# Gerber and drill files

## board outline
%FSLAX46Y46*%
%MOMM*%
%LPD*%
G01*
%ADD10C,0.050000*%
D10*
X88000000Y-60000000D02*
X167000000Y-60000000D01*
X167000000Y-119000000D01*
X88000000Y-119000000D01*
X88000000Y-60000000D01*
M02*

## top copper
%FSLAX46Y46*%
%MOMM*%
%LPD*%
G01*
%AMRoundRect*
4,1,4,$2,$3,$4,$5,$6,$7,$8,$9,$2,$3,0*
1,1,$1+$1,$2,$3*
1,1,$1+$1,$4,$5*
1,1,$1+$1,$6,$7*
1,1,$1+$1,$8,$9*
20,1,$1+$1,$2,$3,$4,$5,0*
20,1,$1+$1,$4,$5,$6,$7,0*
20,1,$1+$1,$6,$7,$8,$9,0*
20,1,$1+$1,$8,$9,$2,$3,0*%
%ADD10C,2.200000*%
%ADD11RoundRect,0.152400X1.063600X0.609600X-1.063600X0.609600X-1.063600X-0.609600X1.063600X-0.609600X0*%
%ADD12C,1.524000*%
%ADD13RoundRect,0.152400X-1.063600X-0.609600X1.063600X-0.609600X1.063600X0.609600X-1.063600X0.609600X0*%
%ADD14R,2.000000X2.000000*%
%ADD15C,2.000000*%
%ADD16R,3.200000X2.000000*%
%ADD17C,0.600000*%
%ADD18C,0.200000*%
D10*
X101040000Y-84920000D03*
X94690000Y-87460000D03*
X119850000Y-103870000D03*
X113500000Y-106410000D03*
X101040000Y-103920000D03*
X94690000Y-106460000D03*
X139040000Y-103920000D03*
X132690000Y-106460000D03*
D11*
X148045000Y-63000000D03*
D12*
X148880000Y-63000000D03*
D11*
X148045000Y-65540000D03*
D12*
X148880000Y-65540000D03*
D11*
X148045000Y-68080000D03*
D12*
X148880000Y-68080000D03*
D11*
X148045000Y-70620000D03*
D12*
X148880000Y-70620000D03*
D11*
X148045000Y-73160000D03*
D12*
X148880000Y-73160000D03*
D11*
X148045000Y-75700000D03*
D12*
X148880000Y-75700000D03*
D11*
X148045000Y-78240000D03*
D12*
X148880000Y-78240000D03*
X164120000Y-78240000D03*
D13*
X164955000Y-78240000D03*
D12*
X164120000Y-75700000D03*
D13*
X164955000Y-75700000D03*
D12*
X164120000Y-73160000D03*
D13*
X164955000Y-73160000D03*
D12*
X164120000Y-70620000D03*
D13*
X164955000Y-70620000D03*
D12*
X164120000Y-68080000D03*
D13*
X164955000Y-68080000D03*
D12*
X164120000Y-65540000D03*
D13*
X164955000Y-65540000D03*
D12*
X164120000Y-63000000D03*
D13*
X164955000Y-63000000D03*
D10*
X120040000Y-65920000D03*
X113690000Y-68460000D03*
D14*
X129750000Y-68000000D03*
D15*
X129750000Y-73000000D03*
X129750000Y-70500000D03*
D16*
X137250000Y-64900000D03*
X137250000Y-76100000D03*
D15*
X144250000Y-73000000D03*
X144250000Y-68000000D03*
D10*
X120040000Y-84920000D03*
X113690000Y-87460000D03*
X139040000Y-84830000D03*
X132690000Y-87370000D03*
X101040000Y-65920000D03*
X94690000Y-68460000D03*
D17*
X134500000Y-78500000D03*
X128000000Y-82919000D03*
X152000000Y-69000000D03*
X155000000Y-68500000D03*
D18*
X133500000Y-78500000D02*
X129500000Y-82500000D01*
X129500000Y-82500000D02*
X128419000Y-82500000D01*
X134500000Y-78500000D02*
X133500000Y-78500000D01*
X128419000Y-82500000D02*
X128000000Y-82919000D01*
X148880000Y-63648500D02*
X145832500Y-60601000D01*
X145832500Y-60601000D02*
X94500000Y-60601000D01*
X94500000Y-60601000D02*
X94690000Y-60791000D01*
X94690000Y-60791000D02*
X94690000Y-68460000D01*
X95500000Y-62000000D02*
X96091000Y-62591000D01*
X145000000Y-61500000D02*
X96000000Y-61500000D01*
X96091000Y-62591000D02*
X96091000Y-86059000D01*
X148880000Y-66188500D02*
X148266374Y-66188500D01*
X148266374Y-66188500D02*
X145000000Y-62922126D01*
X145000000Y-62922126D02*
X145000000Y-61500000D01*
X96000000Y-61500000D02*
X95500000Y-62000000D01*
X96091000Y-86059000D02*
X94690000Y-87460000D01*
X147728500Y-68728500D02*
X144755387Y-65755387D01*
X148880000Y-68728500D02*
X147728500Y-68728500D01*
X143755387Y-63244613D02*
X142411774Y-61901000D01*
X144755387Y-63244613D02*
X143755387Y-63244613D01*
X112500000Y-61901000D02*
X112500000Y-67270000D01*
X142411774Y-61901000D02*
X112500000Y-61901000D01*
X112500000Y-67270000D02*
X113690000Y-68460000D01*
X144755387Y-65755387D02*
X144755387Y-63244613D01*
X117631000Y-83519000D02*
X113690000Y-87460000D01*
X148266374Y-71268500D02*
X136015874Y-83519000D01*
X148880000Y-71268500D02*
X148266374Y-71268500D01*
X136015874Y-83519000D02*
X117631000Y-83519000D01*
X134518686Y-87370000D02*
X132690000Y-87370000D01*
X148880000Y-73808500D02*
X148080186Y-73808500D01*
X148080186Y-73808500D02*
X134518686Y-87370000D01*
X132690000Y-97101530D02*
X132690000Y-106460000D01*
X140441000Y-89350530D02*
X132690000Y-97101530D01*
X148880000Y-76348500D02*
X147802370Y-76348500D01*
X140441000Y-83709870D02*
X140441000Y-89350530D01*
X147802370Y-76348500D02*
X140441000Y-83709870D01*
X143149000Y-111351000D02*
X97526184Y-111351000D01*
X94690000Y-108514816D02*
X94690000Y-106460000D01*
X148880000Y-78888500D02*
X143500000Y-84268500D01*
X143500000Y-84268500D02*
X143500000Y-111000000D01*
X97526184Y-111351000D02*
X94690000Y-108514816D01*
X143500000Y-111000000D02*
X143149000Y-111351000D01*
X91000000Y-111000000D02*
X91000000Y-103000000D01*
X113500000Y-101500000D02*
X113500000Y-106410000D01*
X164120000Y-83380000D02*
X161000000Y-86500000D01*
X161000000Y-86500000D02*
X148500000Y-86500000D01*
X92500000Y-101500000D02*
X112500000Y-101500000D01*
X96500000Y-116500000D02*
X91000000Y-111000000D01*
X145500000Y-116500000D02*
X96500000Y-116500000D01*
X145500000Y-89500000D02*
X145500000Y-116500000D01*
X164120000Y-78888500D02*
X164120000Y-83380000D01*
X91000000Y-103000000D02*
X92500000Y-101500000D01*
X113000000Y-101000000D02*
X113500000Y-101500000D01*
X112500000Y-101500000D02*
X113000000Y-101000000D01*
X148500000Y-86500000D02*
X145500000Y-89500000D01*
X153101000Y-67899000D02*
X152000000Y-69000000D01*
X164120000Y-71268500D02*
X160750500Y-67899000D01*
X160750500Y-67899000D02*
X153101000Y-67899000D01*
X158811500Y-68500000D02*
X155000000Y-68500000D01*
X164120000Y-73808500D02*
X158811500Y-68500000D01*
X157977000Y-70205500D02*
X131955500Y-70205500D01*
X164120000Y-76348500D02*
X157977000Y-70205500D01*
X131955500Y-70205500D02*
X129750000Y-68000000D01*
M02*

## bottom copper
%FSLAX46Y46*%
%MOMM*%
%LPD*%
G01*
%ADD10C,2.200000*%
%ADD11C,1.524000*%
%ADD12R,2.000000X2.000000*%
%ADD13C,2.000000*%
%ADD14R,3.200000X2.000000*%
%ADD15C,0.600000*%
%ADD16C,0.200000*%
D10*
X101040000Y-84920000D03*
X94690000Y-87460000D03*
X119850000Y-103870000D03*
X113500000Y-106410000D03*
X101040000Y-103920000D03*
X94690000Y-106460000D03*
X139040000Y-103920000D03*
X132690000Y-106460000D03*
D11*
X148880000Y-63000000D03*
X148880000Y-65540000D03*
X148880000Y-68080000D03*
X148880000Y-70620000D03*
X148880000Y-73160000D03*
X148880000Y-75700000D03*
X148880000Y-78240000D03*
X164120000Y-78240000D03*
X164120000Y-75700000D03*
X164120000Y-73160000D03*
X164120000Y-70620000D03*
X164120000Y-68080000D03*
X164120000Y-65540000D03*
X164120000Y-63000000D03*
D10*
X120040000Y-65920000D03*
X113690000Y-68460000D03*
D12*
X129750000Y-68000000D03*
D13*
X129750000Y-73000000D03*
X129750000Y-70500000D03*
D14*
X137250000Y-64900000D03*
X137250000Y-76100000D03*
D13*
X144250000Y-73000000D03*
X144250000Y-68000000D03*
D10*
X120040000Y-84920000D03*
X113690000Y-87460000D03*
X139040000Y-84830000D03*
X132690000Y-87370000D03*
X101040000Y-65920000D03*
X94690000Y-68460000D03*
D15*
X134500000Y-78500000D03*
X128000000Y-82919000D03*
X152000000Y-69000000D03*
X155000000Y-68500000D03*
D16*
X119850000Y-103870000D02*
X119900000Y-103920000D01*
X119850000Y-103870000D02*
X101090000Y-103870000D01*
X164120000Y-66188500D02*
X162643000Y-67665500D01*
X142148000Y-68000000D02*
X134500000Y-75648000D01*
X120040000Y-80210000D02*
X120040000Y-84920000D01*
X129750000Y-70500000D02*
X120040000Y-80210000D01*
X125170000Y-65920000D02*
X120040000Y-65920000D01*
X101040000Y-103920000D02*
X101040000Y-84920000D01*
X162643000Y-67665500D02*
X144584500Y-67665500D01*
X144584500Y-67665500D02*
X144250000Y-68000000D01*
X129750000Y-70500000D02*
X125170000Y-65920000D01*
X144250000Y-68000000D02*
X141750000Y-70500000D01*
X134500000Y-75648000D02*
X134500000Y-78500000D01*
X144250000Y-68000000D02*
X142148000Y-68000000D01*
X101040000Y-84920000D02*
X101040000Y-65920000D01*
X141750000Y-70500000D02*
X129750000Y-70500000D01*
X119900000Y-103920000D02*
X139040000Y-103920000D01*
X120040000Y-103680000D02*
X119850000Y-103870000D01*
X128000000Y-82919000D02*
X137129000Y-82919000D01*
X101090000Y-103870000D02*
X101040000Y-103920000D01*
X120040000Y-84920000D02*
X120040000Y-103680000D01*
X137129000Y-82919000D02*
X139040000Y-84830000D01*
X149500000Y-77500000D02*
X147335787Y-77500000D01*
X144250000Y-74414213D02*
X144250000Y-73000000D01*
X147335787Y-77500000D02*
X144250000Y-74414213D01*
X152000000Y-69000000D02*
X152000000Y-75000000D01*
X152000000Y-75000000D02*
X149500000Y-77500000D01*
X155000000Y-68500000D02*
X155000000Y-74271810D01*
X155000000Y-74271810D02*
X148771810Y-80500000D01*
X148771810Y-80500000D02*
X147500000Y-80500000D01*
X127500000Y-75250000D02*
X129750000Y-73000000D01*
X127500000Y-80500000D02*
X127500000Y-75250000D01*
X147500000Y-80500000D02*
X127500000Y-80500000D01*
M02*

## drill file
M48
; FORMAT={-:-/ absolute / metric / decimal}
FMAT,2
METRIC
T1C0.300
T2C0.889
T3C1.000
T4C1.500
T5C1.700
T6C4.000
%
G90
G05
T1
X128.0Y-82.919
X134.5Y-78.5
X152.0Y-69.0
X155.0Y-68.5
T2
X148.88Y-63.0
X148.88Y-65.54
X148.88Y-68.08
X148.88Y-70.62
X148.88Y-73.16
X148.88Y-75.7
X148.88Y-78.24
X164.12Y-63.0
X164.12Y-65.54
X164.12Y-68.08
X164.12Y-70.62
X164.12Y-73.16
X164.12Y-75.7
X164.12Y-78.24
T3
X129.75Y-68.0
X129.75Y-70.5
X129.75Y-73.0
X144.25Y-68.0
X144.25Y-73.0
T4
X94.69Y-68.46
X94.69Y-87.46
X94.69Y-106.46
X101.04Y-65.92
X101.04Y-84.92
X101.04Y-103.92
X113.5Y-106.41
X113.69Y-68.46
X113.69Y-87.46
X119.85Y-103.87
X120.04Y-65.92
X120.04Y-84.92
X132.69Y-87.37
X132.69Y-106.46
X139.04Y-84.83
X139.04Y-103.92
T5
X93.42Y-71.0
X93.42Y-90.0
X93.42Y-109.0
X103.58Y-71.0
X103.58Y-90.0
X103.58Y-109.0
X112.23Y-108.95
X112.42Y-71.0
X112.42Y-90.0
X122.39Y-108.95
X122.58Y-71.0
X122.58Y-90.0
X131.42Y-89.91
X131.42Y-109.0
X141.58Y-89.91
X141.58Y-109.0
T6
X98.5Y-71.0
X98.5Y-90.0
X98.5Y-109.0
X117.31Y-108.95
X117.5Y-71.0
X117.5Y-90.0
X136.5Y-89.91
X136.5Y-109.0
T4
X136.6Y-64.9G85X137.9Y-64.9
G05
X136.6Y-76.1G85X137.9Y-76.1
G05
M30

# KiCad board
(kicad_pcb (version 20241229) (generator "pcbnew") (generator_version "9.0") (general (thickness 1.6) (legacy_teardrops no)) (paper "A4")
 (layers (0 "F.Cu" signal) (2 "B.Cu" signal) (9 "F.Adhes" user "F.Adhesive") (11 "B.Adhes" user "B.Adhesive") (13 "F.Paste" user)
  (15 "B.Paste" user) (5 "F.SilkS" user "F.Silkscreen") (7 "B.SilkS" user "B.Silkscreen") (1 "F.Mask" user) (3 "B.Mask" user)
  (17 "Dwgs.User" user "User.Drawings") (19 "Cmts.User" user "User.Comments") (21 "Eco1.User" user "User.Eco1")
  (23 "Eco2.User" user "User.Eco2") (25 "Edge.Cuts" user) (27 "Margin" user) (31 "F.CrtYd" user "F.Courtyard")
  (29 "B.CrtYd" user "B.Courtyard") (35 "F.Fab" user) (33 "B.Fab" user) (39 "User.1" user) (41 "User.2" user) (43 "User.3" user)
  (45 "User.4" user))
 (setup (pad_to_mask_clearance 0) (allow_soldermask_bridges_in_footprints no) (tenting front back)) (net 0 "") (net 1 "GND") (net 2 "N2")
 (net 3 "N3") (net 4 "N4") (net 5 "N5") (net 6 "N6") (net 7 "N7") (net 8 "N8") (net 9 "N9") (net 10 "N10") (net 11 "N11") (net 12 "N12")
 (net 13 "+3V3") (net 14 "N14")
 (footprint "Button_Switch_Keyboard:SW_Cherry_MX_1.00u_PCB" (layer "F.Cu") (at 101.04 84.92)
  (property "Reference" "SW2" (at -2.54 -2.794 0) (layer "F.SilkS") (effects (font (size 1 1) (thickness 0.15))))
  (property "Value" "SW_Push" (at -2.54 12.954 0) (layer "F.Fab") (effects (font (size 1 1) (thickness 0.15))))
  (pad "" np_thru_hole circle (at -7.62 5.08) (size 1.7 1.7) (drill 1.7) (layers "*.Cu" "*.Mask"))
  (pad "" np_thru_hole circle (at -2.54 5.08) (size 4 4) (drill 4) (layers "*.Cu" "*.Mask"))
  (pad "" np_thru_hole circle (at 2.54 5.08) (size 1.7 1.7) (drill 1.7) (layers "*.Cu" "*.Mask"))
  (pad "1" thru_hole circle (at 0 0) (size 2.2 2.2) (drill 1.5) (layers "*.Cu" "*.Mask") (remove_unused_layers no) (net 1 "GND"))
  (pad "2" thru_hole circle (at -6.35 2.54) (size 2.2 2.2) (drill 1.5) (layers "*.Cu" "*.Mask") (remove_unused_layers no) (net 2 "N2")))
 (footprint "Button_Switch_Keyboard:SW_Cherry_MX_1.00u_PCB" (layer "F.Cu") (at 119.85 103.87)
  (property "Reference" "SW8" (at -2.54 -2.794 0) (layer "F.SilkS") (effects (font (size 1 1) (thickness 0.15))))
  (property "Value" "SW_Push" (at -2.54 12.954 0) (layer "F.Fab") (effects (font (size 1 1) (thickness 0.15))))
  (pad "" np_thru_hole circle (at -7.62 5.08) (size 1.7 1.7) (drill 1.7) (layers "*.Cu" "*.Mask"))
  (pad "" np_thru_hole circle (at -2.54 5.08) (size 4 4) (drill 4) (layers "*.Cu" "*.Mask"))
  (pad "" np_thru_hole circle (at 2.54 5.08) (size 1.7 1.7) (drill 1.7) (layers "*.Cu" "*.Mask"))
  (pad "1" thru_hole circle (at 0 0) (size 2.2 2.2) (drill 1.5) (layers "*.Cu" "*.Mask") (remove_unused_layers no) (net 1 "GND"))
  (pad "2" thru_hole circle (at -6.35 2.54) (size 2.2 2.2) (drill 1.5) (layers "*.Cu" "*.Mask") (remove_unused_layers no) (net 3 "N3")))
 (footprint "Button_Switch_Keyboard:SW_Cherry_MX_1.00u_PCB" (layer "F.Cu") (at 101.04 103.92)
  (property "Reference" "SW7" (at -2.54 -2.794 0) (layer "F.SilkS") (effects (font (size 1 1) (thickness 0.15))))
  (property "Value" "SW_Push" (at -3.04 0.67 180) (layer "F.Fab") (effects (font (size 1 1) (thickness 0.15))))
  (pad "" np_thru_hole circle (at -7.62 5.08) (size 1.7 1.7) (drill 1.7) (layers "*.Cu" "*.Mask"))
  (pad "" np_thru_hole circle (at -2.54 5.08) (size 4 4) (drill 4) (layers "*.Cu" "*.Mask"))
  (pad "" np_thru_hole circle (at 2.54 5.08) (size 1.7 1.7) (drill 1.7) (layers "*.Cu" "*.Mask"))
  (pad "1" thru_hole circle (at 0 0) (size 2.2 2.2) (drill 1.5) (layers "*.Cu" "*.Mask") (remove_unused_layers no) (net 1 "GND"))
  (pad "2" thru_hole circle (at -6.35 2.54) (size 2.2 2.2) (drill 1.5) (layers "*.Cu" "*.Mask") (remove_unused_layers no) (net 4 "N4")))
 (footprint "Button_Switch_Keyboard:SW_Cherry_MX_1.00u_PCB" (layer "F.Cu") (at 139.04 103.92)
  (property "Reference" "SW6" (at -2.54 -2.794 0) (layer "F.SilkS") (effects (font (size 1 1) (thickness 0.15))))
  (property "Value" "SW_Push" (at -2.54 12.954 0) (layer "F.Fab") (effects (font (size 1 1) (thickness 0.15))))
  (pad "" np_thru_hole circle (at -7.62 5.08) (size 1.7 1.7) (drill 1.7) (layers "*.Cu" "*.Mask"))
  (pad "" np_thru_hole circle (at -2.54 5.08) (size 4 4) (drill 4) (layers "*.Cu" "*.Mask"))
  (pad "" np_thru_hole circle (at 2.54 5.08) (size 1.7 1.7) (drill 1.7) (layers "*.Cu" "*.Mask"))
  (pad "1" thru_hole circle (at 0 0) (size 2.2 2.2) (drill 1.5) (layers "*.Cu" "*.Mask") (remove_unused_layers no) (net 1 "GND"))
  (pad "2" thru_hole circle (at -6.35 2.54) (size 2.2 2.2) (drill 1.5) (layers "*.Cu" "*.Mask") (remove_unused_layers no) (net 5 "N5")))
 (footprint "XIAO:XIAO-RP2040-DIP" (layer "F.Cu") (at 156.5 70.62)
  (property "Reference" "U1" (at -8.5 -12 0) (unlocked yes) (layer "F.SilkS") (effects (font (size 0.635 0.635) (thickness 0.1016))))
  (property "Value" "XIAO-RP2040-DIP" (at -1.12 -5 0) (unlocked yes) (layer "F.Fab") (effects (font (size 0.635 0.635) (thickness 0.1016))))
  (pad "1" smd roundrect (at -8.455 -7.62 180) (size 2.432 1.524) (layers "F.Cu" "F.Mask") (roundrect_rratio 0.1) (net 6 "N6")
   (thermal_bridge_angle 45))
  (pad "1" thru_hole circle (at -7.62 -7.62 180) (size 1.524 1.524) (drill 0.889) (layers "*.Cu" "*.Mask") (remove_unused_layers no)
   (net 6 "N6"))
  (pad "2" smd roundrect (at -8.455 -5.08 180) (size 2.432 1.524) (layers "F.Cu" "F.Mask") (roundrect_rratio 0.1) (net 2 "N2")
   (thermal_bridge_angle 45))
  (pad "2" thru_hole circle (at -7.62 -5.08 180) (size 1.524 1.524) (drill 0.889) (layers "*.Cu" "*.Mask") (remove_unused_layers no)
   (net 2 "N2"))
  (pad "3" smd roundrect (at -8.455 -2.54 180) (size 2.432 1.524) (layers "F.Cu" "F.Mask") (roundrect_rratio 0.1) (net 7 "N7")
   (thermal_bridge_angle 45))
  (pad "3" thru_hole circle (at -7.62 -2.54 180) (size 1.524 1.524) (drill 0.889) (layers "*.Cu" "*.Mask") (remove_unused_layers no)
   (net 7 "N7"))
  (pad "4" smd roundrect (at -8.455 0 180) (size 2.432 1.524) (layers "F.Cu" "F.Mask") (roundrect_rratio 0.1) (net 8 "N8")
   (thermal_bridge_angle 45))
  (pad "4" thru_hole circle (at -7.62 0 180) (size 1.524 1.524) (drill 0.889) (layers "*.Cu" "*.Mask") (remove_unused_layers no)
   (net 8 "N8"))
  (pad "5" smd roundrect (at -8.455 2.54 180) (size 2.432 1.524) (layers "F.Cu" "F.Mask") (roundrect_rratio 0.1) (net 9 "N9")
   (thermal_bridge_angle 45))
  (pad "5" thru_hole circle (at -7.62 2.54 180) (size 1.524 1.524) (drill 0.889) (layers "*.Cu" "*.Mask") (remove_unused_layers no)
   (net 9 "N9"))
  (pad "6" smd roundrect (at -8.455 5.08 180) (size 2.432 1.524) (layers "F.Cu" "F.Mask") (roundrect_rratio 0.1) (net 5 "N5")
   (thermal_bridge_angle 45))
  (pad "6" thru_hole circle (at -7.62 5.08 180) (size 1.524 1.524) (drill 0.889) (layers "*.Cu" "*.Mask") (remove_unused_layers no)
   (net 5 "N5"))
  (pad "7" smd roundrect (at -8.455 7.62 180) (size 2.432 1.524) (layers "F.Cu" "F.Mask") (roundrect_rratio 0.1) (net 4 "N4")
   (thermal_bridge_angle 45))
  (pad "7" thru_hole circle (at -7.62 7.62 180) (size 1.524 1.524) (drill 0.889) (layers "*.Cu" "*.Mask") (remove_unused_layers no)
   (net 4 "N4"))
  (pad "8" thru_hole circle (at 7.62 7.62) (size 1.524 1.524) (drill 0.889) (layers "*.Cu" "*.Mask") (remove_unused_layers no) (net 3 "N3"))
  (pad "8" smd roundrect (at 8.455 7.62) (size 2.432 1.524) (layers "F.Cu" "F.Mask") (roundrect_rratio 0.1) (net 3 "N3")
   (thermal_bridge_angle 45))
  (pad "9" thru_hole circle (at 7.62 5.08) (size 1.524 1.524) (drill 0.889) (layers "*.Cu" "*.Mask") (remove_unused_layers no)
   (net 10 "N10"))
  (pad "9" smd roundrect (at 8.455 5.08) (size 2.432 1.524) (layers "F.Cu" "F.Mask") (roundrect_rratio 0.1) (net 10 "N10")
   (thermal_bridge_angle 45))
  (pad "10" thru_hole circle (at 7.62 2.54) (size 1.524 1.524) (drill 0.889) (layers "*.Cu" "*.Mask") (remove_unused_layers no)
   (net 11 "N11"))
  (pad "10" smd roundrect (at 8.455 2.54) (size 2.432 1.524) (layers "F.Cu" "F.Mask") (roundrect_rratio 0.1) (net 11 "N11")
   (thermal_bridge_angle 45))
  (pad "11" thru_hole circle (at 7.62 0) (size 1.524 1.524) (drill 0.889) (layers "*.Cu" "*.Mask") (remove_unused_layers no) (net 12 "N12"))
  (pad "11" smd roundrect (at 8.455 0) (size 2.432 1.524) (layers "F.Cu" "F.Mask") (roundrect_rratio 0.1) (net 12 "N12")
   (thermal_bridge_angle 45))
  (pad "12" thru_hole circle (at 7.62 -2.54) (size 1.524 1.524) (drill 0.889) (layers "*.Cu" "*.Mask") (remove_unused_layers no)
   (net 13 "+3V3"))
  (pad "12" smd roundrect (at 8.455 -2.54) (size 2.432 1.524) (layers "F.Cu" "F.Mask") (roundrect_rratio 0.1) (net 13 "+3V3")
   (thermal_bridge_angle 45))
  (pad "13" thru_hole circle (at 7.62 -5.08) (size 1.524 1.524) (drill 0.889) (layers "*.Cu" "*.Mask") (remove_unused_layers no)
   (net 1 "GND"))
  (pad "13" smd roundrect (at 8.455 -5.08) (size 2.432 1.524) (layers "F.Cu" "F.Mask") (roundrect_rratio 0.1) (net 1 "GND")
   (thermal_bridge_angle 45))
  (pad "14" thru_hole circle (at 7.62 -7.62) (size 1.524 1.524) (drill 0.889) (layers "*.Cu" "*.Mask") (remove_unused_layers no)
   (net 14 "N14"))
  (pad "14" smd roundrect (at 8.455 -7.62) (size 2.432 1.524) (layers "F.Cu" "F.Mask") (roundrect_rratio 0.1) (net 14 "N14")
   (thermal_bridge_angle 45)))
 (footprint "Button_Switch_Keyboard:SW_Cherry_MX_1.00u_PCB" (layer "F.Cu") (at 120.04 65.92)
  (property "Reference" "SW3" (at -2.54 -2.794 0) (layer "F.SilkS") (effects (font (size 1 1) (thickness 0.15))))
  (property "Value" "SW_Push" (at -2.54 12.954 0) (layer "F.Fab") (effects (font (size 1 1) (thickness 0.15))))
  (pad "" np_thru_hole circle (at -7.62 5.08) (size 1.7 1.7) (drill 1.7) (layers "*.Cu" "*.Mask"))
  (pad "" np_thru_hole circle (at -2.54 5.08) (size 4 4) (drill 4) (layers "*.Cu" "*.Mask"))
  (pad "" np_thru_hole circle (at 2.54 5.08) (size 1.7 1.7) (drill 1.7) (layers "*.Cu" "*.Mask"))
  (pad "1" thru_hole circle (at 0 0) (size 2.2 2.2) (drill 1.5) (layers "*.Cu" "*.Mask") (remove_unused_layers no) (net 1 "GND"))
  (pad "2" thru_hole circle (at -6.35 2.54) (size 2.2 2.2) (drill 1.5) (layers "*.Cu" "*.Mask") (remove_unused_layers no) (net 7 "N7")))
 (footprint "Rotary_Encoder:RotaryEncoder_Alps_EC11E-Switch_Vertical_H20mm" (layer "F.Cu") (at 129.75 68)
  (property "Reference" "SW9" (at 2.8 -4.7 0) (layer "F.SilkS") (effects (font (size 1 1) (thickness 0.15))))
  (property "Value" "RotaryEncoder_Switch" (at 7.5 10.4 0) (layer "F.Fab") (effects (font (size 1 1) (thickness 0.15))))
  (pad "A" thru_hole rect (at 0 0) (size 2 2) (drill 1) (layers "*.Cu" "*.Mask") (remove_unused_layers no) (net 10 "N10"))
  (pad "B" thru_hole circle (at 0 5) (size 2 2) (drill 1) (layers "*.Cu" "*.Mask") (remove_unused_layers no) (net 11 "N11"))
  (pad "C" thru_hole circle (at 0 2.5) (size 2 2) (drill 1) (layers "*.Cu" "*.Mask") (remove_unused_layers no) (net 1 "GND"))
  (pad "MP" thru_hole rect (at 7.5 -3.1) (size 3.2 2) (drill oval 2.8 1.5) (layers "*.Cu" "*.Mask") (remove_unused_layers no))
  (pad "MP" thru_hole rect (at 7.5 8.1) (size 3.2 2) (drill oval 2.8 1.5) (layers "*.Cu" "*.Mask") (remove_unused_layers no))
  (pad "S1" thru_hole circle (at 14.5 5) (size 2 2) (drill 1) (layers "*.Cu" "*.Mask") (remove_unused_layers no) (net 12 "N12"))
  (pad "S2" thru_hole circle (at 14.5 0) (size 2 2) (drill 1) (layers "*.Cu" "*.Mask") (remove_unused_layers no) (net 1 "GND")))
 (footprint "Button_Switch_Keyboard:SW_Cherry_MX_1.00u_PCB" (layer "F.Cu") (at 120.04 84.92)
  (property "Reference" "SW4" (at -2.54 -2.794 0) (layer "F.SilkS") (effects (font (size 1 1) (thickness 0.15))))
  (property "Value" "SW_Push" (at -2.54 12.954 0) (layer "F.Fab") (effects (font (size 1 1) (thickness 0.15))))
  (pad "" np_thru_hole circle (at -7.62 5.08) (size 1.7 1.7) (drill 1.7) (layers "*.Cu" "*.Mask"))
  (pad "" np_thru_hole circle (at -2.54 5.08) (size 4 4) (drill 4) (layers "*.Cu" "*.Mask"))
  (pad "" np_thru_hole circle (at 2.54 5.08) (size 1.7 1.7) (drill 1.7) (layers "*.Cu" "*.Mask"))
  (pad "1" thru_hole circle (at 0 0) (size 2.2 2.2) (drill 1.5) (layers "*.Cu" "*.Mask") (remove_unused_layers no) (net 1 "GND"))
  (pad "2" thru_hole circle (at -6.35 2.54) (size 2.2 2.2) (drill 1.5) (layers "*.Cu" "*.Mask") (remove_unused_layers no) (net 8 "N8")))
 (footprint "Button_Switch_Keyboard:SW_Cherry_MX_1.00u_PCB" (layer "F.Cu") (at 139.04 84.83)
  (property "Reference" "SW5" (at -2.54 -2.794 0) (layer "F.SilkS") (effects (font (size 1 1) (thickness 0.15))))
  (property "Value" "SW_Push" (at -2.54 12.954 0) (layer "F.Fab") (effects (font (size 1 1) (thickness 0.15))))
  (pad "" np_thru_hole circle (at -7.62 5.08) (size 1.7 1.7) (drill 1.7) (layers "*.Cu" "*.Mask"))
  (pad "" np_thru_hole circle (at -2.54 5.08) (size 4 4) (drill 4) (layers "*.Cu" "*.Mask"))
  (pad "" np_thru_hole circle (at 2.54 5.08) (size 1.7 1.7) (drill 1.7) (layers "*.Cu" "*.Mask"))
  (pad "1" thru_hole circle (at 0 0) (size 2.2 2.2) (drill 1.5) (layers "*.Cu" "*.Mask") (remove_unused_layers no) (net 1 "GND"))
  (pad "2" thru_hole circle (at -6.35 2.54) (size 2.2 2.2) (drill 1.5) (layers "*.Cu" "*.Mask") (remove_unused_layers no) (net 9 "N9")))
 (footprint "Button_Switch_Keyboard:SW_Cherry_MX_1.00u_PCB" (layer "F.Cu") (at 101.04 65.92)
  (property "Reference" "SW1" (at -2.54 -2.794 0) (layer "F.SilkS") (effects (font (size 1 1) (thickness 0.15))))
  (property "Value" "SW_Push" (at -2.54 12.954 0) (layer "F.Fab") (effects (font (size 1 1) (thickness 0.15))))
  (pad "" np_thru_hole circle (at -7.62 5.08) (size 1.7 1.7) (drill 1.7) (layers "*.Cu" "*.Mask"))
  (pad "" np_thru_hole circle (at -2.54 5.08) (size 4 4) (drill 4) (layers "*.Cu" "*.Mask"))
  (pad "" np_thru_hole circle (at 2.54 5.08) (size 1.7 1.7) (drill 1.7) (layers "*.Cu" "*.Mask"))
  (pad "1" thru_hole circle (at 0 0) (size 2.2 2.2) (drill 1.5) (layers "*.Cu" "*.Mask") (remove_unused_layers no) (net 1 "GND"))
  (pad "2" thru_hole circle (at -6.35 2.54) (size 2.2 2.2) (drill 1.5) (layers "*.Cu" "*.Mask") (remove_unused_layers no) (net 6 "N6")))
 (gr_rect (start 88 60) (end 167 119) (stroke (width 0.05) (type default)) (fill no) (layer "Edge.Cuts"))
 (segment (start 133.5 78.5) (end 129.5 82.5) (width 0.2) (layer "F.Cu") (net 1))
 (segment (start 129.5 82.5) (end 128.419 82.5) (width 0.2) (layer "F.Cu") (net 1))
 (segment (start 134.5 78.5) (end 133.5 78.5) (width 0.2) (layer "F.Cu") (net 1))
 (segment (start 128.419 82.5) (end 128 82.919) (width 0.2) (layer "F.Cu") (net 1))
 (via (at 134.5 78.5) (size 0.6) (drill 0.3) (layers "F.Cu" "B.Cu") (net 1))
 (via (at 128 82.919) (size 0.6) (drill 0.3) (layers "F.Cu" "B.Cu") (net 1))
 (segment (start 119.85 103.87) (end 119.9 103.92) (width 0.2) (layer "B.Cu") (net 1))
 (segment (start 119.85 103.87) (end 101.09 103.87) (width 0.2) (layer "B.Cu") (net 1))
 (segment (start 164.12 66.1885) (end 162.643 67.6655) (width 0.2) (layer "B.Cu") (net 1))
 (segment (start 142.148 68) (end 134.5 75.648) (width 0.2) (layer "B.Cu") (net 1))
 (segment (start 120.04 80.21) (end 120.04 84.92) (width 0.2) (layer "B.Cu") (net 1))
 (segment (start 129.75 70.5) (end 120.04 80.21) (width 0.2) (layer "B.Cu") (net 1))
 (segment (start 125.17 65.92) (end 120.04 65.92) (width 0.2) (layer "B.Cu") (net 1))
 (segment (start 101.04 103.92) (end 101.04 84.92) (width 0.2) (layer "B.Cu") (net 1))
 (segment (start 162.643 67.6655) (end 144.5845 67.6655) (width 0.2) (layer "B.Cu") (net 1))
 (segment (start 144.5845 67.6655) (end 144.25 68) (width 0.2) (layer "B.Cu") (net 1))
 (segment (start 129.75 70.5) (end 125.17 65.92) (width 0.2) (layer "B.Cu") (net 1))
 (segment (start 144.25 68) (end 141.75 70.5) (width 0.2) (layer "B.Cu") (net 1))
 (segment (start 134.5 75.648) (end 134.5 78.5) (width 0.2) (layer "B.Cu") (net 1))
 (segment (start 144.25 68) (end 142.148 68) (width 0.2) (layer "B.Cu") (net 1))
 (segment (start 101.04 84.92) (end 101.04 65.92) (width 0.2) (layer "B.Cu") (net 1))
 (segment (start 141.75 70.5) (end 129.75 70.5) (width 0.2) (layer "B.Cu") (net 1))
 (segment (start 119.9 103.92) (end 139.04 103.92) (width 0.2) (layer "B.Cu") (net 1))
 (segment (start 120.04 103.68) (end 119.85 103.87) (width 0.2) (layer "B.Cu") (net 1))
 (segment (start 128 82.919) (end 137.129 82.919) (width 0.2) (layer "B.Cu") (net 1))
 (segment (start 101.09 103.87) (end 101.04 103.92) (width 0.2) (layer "B.Cu") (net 1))
 (segment (start 120.04 84.92) (end 120.04 103.68) (width 0.2) (layer "B.Cu") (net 1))
 (segment (start 137.129 82.919) (end 139.04 84.83) (width 0.2) (layer "B.Cu") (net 1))
 (segment (start 148.88 63.6485) (end 145.8325 60.601) (width 0.2) (layer "F.Cu") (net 6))
 (segment (start 145.8325 60.601) (end 94.5 60.601) (width 0.2) (layer "F.Cu") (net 6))
 (segment (start 94.5 60.601) (end 94.69 60.791) (width 0.2) (layer "F.Cu") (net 6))
 (segment (start 94.69 60.791) (end 94.69 68.46) (width 0.2) (layer "F.Cu") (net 6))
 (segment (start 95.5 62) (end 96.091 62.591) (width 0.2) (layer "F.Cu") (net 2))
 (segment (start 145 61.5) (end 96 61.5) (width 0.2) (layer "F.Cu") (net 2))
 (segment (start 96.091 62.591) (end 96.091 86.059) (width 0.2) (layer "F.Cu") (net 2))
 (segment (start 148.88 66.1885) (end 148.266374 66.1885) (width 0.2) (layer "F.Cu") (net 2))
 (segment (start 148.266374 66.1885) (end 145 62.922126) (width 0.2) (layer "F.Cu") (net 2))
 (segment (start 145 62.922126) (end 145 61.5) (width 0.2) (layer "F.Cu") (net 2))
 (segment (start 96 61.5) (end 95.5 62) (width 0.2) (layer "F.Cu") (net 2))
 (segment (start 96.091 86.059) (end 94.69 87.46) (width 0.2) (layer "F.Cu") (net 2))
 (segment (start 147.7285 68.7285) (end 144.755387 65.755387) (width 0.2) (layer "F.Cu") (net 7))
 (segment (start 148.88 68.7285) (end 147.7285 68.7285) (width 0.2) (layer "F.Cu") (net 7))
 (segment (start 143.755387 63.244613) (end 142.411774 61.901) (width 0.2) (layer "F.Cu") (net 7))
 (segment (start 144.755387 63.244613) (end 143.755387 63.244613) (width 0.2) (layer "F.Cu") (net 7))
 (segment (start 112.5 61.901) (end 112.5 67.27) (width 0.2) (layer "F.Cu") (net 7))
 (segment (start 142.411774 61.901) (end 112.5 61.901) (width 0.2) (layer "F.Cu") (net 7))
 (segment (start 112.5 67.27) (end 113.69 68.46) (width 0.2) (layer "F.Cu") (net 7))
 (segment (start 144.755387 65.755387) (end 144.755387 63.244613) (width 0.2) (layer "F.Cu") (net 7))
 (segment (start 117.631 83.519) (end 113.69 87.46) (width 0.2) (layer "F.Cu") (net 8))
 (segment (start 148.266374 71.2685) (end 136.015874 83.519) (width 0.2) (layer "F.Cu") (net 8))
 (segment (start 148.88 71.2685) (end 148.266374 71.2685) (width 0.2) (layer "F.Cu") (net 8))
 (segment (start 136.015874 83.519) (end 117.631 83.519) (width 0.2) (layer "F.Cu") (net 8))
 (segment (start 134.518686 87.37) (end 132.69 87.37) (width 0.2) (layer "F.Cu") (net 9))
 (segment (start 148.88 73.8085) (end 148.080186 73.8085) (width 0.2) (layer "F.Cu") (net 9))
 (segment (start 148.080186 73.8085) (end 134.518686 87.37) (width 0.2) (layer "F.Cu") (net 9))
 (segment (start 132.69 97.10153) (end 132.69 106.46) (width 0.2) (layer "F.Cu") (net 5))
 (segment (start 140.441 89.35053) (end 132.69 97.10153) (width 0.2) (layer "F.Cu") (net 5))
 (segment (start 148.88 76.3485) (end 147.80237 76.3485) (width 0.2) (layer "F.Cu") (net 5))
 (segment (start 140.441 83.70987) (end 140.441 89.35053) (width 0.2) (layer "F.Cu") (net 5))
 (segment (start 147.80237 76.3485) (end 140.441 83.70987) (width 0.2) (layer "F.Cu") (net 5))
 (segment (start 143.149 111.351) (end 97.526184 111.351) (width 0.2) (layer "F.Cu") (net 4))
 (segment (start 94.69 108.514816) (end 94.69 106.46) (width 0.2) (layer "F.Cu") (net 4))
 (segment (start 148.88 78.8885) (end 143.5 84.2685) (width 0.2) (layer "F.Cu") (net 4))
 (segment (start 143.5 84.2685) (end 143.5 111) (width 0.2) (layer "F.Cu") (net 4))
 (segment (start 97.526184 111.351) (end 94.69 108.514816) (width 0.2) (layer "F.Cu") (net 4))
 (segment (start 143.5 111) (end 143.149 111.351) (width 0.2) (layer "F.Cu") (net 4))
 (segment (start 91 111) (end 91 103) (width 0.2) (layer "F.Cu") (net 3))
 (segment (start 113.5 101.5) (end 113.5 106.41) (width 0.2) (layer "F.Cu") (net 3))
 (segment (start 164.12 83.38) (end 161 86.5) (width 0.2) (layer "F.Cu") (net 3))
 (segment (start 161 86.5) (end 148.5 86.5) (width 0.2) (layer "F.Cu") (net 3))
 (segment (start 92.5 101.5) (end 112.5 101.5) (width 0.2) (layer "F.Cu") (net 3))
 (segment (start 96.5 116.5) (end 91 111) (width 0.2) (layer "F.Cu") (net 3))
 (segment (start 145.5 116.5) (end 96.5 116.5) (width 0.2) (layer "F.Cu") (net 3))
 (segment (start 145.5 89.5) (end 145.5 116.5) (width 0.2) (layer "F.Cu") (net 3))
 (segment (start 164.12 78.8885) (end 164.12 83.38) (width 0.2) (layer "F.Cu") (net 3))
 (segment (start 91 103) (end 92.5 101.5) (width 0.2) (layer "F.Cu") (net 3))
 (segment (start 113 101) (end 113.5 101.5) (width 0.2) (layer "F.Cu") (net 3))
 (segment (start 112.5 101.5) (end 113 101) (width 0.2) (layer "F.Cu") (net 3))
 (segment (start 148.5 86.5) (end 145.5 89.5) (width 0.2) (layer "F.Cu") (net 3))
 (segment (start 153.101 67.899) (end 152 69) (width 0.2) (layer "F.Cu") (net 12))
 (segment (start 164.12 71.2685) (end 160.7505 67.899) (width 0.2) (layer "F.Cu") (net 12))
 (segment (start 160.7505 67.899) (end 153.101 67.899) (width 0.2) (layer "F.Cu") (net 12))
 (via (at 152 69) (size 0.6) (drill 0.3) (layers "F.Cu" "B.Cu") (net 12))
 (segment (start 149.5 77.5) (end 147.335787 77.5) (width 0.2) (layer "B.Cu") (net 12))
 (segment (start 144.25 74.414213) (end 144.25 73) (width 0.2) (layer "B.Cu") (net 12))
 (segment (start 147.335787 77.5) (end 144.25 74.414213) (width 0.2) (layer "B.Cu") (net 12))
 (segment (start 152 69) (end 152 75) (width 0.2) (layer "B.Cu") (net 12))
 (segment (start 152 75) (end 149.5 77.5) (width 0.2) (layer "B.Cu") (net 12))
 (segment (start 158.8115 68.5) (end 155 68.5) (width 0.2) (layer "F.Cu") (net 11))
 (segment (start 164.12 73.8085) (end 158.8115 68.5) (width 0.2) (layer "F.Cu") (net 11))
 (via (at 155 68.5) (size 0.6) (drill 0.3) (layers "F.Cu" "B.Cu") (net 11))
 (segment (start 155 68.5) (end 155 74.27181) (width 0.2) (layer "B.Cu") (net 11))
 (segment (start 155 74.27181) (end 148.77181 80.5) (width 0.2) (layer "B.Cu") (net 11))
 (segment (start 148.77181 80.5) (end 147.5 80.5) (width 0.2) (layer "B.Cu") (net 11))
 (segment (start 127.5 75.25) (end 129.75 73) (width 0.2) (layer "B.Cu") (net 11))
 (segment (start 127.5 80.5) (end 127.5 75.25) (width 0.2) (layer "B.Cu") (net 11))
 (segment (start 147.5 80.5) (end 127.5 80.5) (width 0.2) (layer "B.Cu") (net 11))
 (segment (start 157.977 70.2055) (end 131.9555 70.2055) (width 0.2) (layer "F.Cu") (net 10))
 (segment (start 164.12 76.3485) (end 157.977 70.2055) (width 0.2) (layer "F.Cu") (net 10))
 (segment (start 131.9555 70.2055) (end 129.75 68) (width 0.2) (layer "F.Cu") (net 10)))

